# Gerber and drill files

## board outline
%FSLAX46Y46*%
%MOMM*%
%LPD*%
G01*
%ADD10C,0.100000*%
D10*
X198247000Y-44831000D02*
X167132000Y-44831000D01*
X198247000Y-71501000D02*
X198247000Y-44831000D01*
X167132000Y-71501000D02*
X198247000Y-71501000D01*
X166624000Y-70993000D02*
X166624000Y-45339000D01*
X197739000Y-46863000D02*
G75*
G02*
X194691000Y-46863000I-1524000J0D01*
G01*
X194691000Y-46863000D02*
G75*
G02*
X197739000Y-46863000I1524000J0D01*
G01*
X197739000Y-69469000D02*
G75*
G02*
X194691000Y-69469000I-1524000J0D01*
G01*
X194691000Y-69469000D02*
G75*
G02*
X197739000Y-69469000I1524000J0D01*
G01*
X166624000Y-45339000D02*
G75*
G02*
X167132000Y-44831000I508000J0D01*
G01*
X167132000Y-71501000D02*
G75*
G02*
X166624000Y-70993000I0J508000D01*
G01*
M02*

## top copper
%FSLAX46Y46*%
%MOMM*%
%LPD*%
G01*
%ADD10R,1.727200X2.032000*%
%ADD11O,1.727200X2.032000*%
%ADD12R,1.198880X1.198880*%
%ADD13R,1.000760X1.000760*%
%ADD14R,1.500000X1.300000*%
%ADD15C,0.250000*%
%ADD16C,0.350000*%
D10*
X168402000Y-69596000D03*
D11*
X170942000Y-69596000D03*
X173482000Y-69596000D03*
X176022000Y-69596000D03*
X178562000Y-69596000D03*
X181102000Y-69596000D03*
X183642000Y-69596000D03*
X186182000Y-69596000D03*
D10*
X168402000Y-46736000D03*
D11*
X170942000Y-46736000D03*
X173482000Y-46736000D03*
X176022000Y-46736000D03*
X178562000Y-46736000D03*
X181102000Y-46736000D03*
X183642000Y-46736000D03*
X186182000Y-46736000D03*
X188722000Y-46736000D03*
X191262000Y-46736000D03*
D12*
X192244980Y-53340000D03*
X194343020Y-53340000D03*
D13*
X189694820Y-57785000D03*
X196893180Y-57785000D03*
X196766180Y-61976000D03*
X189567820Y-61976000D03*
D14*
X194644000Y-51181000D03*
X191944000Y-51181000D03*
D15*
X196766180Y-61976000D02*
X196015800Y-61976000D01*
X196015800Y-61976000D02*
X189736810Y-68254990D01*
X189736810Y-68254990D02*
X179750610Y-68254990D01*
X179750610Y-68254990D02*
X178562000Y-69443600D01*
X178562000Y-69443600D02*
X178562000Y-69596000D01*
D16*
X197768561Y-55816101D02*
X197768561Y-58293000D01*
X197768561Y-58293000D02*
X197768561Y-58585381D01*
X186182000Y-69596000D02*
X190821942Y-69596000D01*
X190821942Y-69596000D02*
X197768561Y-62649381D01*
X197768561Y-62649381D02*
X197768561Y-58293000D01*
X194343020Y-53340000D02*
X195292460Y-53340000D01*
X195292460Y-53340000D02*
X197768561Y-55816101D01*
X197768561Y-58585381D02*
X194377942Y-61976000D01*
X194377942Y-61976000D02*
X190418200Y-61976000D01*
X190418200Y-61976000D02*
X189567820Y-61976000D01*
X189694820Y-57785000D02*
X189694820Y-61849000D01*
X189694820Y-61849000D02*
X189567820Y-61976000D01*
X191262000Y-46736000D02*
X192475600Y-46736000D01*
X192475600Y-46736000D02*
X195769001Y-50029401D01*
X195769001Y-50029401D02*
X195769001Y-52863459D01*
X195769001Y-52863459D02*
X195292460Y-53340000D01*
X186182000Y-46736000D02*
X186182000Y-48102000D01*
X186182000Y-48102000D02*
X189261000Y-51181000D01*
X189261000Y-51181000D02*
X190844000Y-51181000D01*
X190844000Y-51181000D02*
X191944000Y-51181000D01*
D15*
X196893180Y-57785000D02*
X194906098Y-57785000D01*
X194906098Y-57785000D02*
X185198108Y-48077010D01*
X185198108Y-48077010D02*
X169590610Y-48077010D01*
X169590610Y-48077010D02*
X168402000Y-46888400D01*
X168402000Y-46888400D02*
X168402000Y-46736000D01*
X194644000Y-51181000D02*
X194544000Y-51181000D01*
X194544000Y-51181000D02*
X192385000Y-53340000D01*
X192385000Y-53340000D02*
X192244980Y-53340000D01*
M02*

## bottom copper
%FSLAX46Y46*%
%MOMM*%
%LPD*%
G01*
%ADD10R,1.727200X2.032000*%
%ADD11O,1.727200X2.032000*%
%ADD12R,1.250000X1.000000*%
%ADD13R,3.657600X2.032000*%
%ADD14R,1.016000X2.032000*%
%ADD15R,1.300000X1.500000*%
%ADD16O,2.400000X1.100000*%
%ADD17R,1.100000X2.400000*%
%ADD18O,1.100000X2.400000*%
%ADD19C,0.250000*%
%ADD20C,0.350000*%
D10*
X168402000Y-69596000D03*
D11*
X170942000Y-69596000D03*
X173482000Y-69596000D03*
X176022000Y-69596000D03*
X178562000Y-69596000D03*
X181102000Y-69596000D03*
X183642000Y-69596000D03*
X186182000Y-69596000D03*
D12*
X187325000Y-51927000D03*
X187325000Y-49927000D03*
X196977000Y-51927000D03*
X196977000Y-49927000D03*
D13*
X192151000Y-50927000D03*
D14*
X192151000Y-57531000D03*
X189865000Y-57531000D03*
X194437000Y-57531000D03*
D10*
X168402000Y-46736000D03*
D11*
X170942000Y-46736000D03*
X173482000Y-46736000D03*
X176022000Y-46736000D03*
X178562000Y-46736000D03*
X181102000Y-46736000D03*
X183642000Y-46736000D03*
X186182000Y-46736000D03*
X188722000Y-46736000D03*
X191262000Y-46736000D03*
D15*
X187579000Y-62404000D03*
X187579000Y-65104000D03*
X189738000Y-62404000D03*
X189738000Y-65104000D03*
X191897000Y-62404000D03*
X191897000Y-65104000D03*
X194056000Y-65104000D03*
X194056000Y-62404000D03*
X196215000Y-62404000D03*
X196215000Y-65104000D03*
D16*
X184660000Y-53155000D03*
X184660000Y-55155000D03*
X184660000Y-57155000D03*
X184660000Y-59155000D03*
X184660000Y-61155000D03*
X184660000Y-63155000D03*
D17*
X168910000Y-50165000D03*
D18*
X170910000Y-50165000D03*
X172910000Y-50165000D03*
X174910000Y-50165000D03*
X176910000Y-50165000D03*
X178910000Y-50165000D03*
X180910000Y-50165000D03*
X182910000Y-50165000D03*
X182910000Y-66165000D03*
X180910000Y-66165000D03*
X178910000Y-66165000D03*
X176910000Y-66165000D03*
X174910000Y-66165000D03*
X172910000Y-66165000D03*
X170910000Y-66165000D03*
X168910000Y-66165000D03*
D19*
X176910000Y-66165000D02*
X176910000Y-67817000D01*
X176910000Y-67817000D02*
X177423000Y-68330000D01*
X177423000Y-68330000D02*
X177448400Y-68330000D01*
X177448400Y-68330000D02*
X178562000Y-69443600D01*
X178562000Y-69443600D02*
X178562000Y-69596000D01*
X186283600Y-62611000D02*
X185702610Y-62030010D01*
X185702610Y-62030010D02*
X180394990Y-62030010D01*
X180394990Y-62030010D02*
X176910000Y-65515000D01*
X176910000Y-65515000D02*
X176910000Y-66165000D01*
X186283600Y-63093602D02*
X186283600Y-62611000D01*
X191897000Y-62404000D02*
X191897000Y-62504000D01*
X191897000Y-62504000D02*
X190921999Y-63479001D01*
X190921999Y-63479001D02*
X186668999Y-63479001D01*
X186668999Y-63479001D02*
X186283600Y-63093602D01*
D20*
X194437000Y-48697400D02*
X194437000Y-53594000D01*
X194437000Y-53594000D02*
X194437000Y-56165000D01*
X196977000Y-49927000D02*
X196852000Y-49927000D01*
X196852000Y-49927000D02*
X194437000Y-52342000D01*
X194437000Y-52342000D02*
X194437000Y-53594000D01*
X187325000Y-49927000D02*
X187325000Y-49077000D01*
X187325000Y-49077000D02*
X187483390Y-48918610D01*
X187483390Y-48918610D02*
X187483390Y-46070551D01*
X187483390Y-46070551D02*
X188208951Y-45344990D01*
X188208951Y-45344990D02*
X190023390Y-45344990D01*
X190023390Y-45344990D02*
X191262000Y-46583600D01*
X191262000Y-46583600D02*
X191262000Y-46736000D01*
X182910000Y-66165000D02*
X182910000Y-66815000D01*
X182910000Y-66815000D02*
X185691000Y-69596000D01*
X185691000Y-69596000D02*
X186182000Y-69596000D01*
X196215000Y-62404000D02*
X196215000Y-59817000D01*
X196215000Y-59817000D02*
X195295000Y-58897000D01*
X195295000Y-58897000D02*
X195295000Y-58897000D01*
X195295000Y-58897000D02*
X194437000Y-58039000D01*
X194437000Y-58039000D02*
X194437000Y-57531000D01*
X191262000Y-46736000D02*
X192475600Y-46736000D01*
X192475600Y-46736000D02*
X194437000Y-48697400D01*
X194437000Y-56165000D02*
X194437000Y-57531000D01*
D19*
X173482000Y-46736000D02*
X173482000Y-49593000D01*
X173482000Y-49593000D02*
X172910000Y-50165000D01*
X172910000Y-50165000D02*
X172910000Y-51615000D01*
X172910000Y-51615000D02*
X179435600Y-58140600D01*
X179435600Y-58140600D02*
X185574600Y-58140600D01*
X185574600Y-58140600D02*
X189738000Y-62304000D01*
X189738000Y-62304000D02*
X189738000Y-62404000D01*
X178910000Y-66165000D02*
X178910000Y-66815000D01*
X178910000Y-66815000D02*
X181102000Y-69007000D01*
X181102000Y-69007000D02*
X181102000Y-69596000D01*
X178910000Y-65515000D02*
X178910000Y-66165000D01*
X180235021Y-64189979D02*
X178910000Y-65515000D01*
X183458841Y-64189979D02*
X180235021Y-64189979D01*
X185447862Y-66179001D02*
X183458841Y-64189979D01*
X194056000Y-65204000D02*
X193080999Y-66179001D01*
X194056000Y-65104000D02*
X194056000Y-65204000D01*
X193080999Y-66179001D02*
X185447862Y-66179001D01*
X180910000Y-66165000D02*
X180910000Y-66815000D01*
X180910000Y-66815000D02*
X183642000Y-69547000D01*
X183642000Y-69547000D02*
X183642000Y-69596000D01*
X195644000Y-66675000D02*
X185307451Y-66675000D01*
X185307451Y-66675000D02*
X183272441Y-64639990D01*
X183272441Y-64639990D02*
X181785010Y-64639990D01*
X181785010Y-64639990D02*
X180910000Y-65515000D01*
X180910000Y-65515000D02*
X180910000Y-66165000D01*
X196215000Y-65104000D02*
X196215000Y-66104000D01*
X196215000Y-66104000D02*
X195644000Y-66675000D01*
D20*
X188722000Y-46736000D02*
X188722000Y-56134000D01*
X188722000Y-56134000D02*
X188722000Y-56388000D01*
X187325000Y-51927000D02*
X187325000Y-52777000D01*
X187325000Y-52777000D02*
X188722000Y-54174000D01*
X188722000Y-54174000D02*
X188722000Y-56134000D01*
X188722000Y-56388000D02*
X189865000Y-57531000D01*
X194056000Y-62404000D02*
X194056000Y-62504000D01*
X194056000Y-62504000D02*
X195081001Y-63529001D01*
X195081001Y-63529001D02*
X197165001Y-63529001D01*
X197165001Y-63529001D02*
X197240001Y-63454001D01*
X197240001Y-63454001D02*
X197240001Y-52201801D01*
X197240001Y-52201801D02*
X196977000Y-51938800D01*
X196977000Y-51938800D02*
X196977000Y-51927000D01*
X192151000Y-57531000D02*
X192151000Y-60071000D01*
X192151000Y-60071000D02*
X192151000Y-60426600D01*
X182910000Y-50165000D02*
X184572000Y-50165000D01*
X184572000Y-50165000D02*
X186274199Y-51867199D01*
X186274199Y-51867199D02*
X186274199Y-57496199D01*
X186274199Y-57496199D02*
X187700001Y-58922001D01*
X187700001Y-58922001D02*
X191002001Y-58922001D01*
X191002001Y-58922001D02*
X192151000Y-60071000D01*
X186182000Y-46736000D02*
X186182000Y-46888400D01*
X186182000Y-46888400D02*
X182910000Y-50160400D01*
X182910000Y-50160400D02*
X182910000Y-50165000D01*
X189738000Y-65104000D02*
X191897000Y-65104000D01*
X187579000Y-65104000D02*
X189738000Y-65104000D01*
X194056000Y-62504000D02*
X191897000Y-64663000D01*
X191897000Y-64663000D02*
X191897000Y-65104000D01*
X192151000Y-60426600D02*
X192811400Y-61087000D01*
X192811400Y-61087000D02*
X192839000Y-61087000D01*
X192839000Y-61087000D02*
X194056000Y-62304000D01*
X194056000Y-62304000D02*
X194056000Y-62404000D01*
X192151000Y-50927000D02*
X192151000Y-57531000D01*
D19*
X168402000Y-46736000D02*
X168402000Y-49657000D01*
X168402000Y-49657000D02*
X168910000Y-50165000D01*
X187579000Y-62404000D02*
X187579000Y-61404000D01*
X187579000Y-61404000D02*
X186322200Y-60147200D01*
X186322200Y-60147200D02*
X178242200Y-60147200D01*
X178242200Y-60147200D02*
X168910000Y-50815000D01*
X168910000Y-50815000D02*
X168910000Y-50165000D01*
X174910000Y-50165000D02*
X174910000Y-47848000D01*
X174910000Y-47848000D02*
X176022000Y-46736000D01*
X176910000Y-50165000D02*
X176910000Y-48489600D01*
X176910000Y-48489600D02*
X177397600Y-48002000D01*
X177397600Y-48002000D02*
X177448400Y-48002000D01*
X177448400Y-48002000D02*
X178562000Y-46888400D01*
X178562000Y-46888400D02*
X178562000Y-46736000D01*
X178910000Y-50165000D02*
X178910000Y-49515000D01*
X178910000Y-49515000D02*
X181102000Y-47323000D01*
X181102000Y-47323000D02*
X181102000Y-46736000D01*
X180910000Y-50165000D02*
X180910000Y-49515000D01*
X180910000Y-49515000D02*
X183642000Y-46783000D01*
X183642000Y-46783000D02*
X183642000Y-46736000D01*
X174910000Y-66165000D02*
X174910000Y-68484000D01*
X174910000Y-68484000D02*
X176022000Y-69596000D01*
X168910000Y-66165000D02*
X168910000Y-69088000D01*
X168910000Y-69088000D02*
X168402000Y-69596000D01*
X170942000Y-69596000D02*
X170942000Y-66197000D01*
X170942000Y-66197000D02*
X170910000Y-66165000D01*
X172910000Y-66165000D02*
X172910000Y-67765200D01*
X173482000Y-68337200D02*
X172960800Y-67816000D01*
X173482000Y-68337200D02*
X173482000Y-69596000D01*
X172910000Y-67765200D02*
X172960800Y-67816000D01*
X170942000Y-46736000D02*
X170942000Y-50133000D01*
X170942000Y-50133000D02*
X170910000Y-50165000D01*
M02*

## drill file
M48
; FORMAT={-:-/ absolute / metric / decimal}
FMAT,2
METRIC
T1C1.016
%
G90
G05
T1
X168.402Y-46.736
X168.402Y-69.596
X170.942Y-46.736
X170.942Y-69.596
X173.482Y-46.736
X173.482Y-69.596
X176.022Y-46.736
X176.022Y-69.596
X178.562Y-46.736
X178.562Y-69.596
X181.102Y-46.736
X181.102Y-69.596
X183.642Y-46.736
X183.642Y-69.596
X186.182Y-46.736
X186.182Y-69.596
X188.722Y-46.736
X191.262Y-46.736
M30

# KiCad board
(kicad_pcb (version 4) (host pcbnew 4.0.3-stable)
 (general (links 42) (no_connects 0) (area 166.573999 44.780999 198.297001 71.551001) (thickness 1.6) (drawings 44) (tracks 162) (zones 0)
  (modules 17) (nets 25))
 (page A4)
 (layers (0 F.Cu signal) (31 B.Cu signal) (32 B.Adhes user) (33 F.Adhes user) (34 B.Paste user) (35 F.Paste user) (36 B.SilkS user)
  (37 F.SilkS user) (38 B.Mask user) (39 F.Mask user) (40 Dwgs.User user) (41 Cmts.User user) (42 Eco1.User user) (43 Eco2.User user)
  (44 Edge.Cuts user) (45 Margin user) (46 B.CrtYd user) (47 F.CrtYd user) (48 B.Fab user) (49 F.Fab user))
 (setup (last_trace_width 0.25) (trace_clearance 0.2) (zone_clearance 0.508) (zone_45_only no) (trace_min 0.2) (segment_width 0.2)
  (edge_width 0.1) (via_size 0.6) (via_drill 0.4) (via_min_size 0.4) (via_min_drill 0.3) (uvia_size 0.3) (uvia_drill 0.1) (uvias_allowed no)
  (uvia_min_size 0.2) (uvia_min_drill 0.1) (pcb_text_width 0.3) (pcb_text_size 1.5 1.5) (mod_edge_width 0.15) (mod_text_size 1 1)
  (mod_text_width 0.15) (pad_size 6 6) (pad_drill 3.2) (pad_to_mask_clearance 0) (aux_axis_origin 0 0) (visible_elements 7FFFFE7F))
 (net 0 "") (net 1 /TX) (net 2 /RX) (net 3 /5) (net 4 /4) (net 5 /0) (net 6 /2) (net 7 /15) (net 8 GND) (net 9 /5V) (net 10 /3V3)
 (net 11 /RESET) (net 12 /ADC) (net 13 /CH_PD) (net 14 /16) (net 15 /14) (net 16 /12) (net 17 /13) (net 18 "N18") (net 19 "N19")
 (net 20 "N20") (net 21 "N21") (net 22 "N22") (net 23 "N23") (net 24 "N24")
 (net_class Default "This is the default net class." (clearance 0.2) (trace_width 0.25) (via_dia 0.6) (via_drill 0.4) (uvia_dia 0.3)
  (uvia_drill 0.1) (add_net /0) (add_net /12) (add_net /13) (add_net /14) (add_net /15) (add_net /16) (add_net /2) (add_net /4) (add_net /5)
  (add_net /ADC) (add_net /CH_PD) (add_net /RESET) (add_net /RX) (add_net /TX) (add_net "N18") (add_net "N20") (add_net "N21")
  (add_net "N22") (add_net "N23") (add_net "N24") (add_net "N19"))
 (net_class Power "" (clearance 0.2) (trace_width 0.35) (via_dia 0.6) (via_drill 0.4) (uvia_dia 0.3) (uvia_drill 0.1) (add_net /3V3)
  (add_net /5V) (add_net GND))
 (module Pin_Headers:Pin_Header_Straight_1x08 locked (layer B.Cu) (at 168.402 69.596 270)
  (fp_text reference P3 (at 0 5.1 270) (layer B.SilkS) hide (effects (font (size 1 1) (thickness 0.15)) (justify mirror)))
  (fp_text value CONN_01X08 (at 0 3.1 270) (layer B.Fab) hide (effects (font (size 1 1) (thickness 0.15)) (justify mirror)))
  (pad 1 thru_hole rect (at 0 0 270) (size 2.032 1.7272) (drill 1.016) (layers *.Cu *.Mask B.SilkS) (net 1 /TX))
  (pad 2 thru_hole oval (at 0 -2.54 270) (size 2.032 1.7272) (drill 1.016) (layers *.Cu *.Mask B.SilkS) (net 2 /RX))
  (pad 3 thru_hole oval (at 0 -5.08 270) (size 2.032 1.7272) (drill 1.016) (layers *.Cu *.Mask B.SilkS) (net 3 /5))
  (pad 4 thru_hole oval (at 0 -7.62 270) (size 2.032 1.7272) (drill 1.016) (layers *.Cu *.Mask B.SilkS) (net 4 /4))
  (pad 5 thru_hole oval (at 0 -10.16 270) (size 2.032 1.7272) (drill 1.016) (layers *.Cu *.Mask B.SilkS) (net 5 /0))
  (pad 6 thru_hole oval (at 0 -12.7 270) (size 2.032 1.7272) (drill 1.016) (layers *.Cu *.Mask B.SilkS) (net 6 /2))
  (pad 7 thru_hole oval (at 0 -15.24 270) (size 2.032 1.7272) (drill 1.016) (layers *.Cu *.Mask B.SilkS) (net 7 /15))
  (pad 8 thru_hole oval (at 0 -17.78 270) (size 2.032 1.7272) (drill 1.016) (layers *.Cu *.Mask B.SilkS) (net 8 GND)))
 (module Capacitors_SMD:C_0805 (layer B.Cu) (at 187.325 50.927 90)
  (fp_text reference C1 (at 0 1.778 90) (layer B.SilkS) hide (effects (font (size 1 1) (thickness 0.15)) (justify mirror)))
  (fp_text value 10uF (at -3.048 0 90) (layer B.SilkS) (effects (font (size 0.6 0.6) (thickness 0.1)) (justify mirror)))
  (pad 1 smd rect (at -1 0 90) (size 1 1.25) (layers B.Cu B.Paste B.Mask) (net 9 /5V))
  (pad 2 smd rect (at 1 0 90) (size 1 1.25) (layers B.Cu B.Paste B.Mask) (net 8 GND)))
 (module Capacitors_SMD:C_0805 (layer B.Cu) (at 196.977 50.927 90)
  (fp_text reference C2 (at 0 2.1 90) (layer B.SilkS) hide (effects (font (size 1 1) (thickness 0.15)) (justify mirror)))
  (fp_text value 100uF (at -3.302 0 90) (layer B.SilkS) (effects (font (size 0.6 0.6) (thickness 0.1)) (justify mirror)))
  (pad 1 smd rect (at -1 0 90) (size 1 1.25) (layers B.Cu B.Paste B.Mask) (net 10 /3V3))
  (pad 2 smd rect (at 1 0 90) (size 1 1.25) (layers B.Cu B.Paste B.Mask) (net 8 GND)))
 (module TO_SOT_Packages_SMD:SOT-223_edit (layer B.Cu) (at 192.151 54.229 180)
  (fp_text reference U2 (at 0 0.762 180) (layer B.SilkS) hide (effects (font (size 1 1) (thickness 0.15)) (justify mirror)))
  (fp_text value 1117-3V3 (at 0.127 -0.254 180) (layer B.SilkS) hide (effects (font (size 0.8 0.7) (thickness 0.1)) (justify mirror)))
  (pad 2 smd rect (at 0 3.302 180) (size 3.6576 2.032) (layers B.Cu B.Paste B.Mask) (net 10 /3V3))
  (pad 2 smd rect (at 0 -3.302 180) (size 1.016 2.032) (layers B.Cu B.Paste B.Mask) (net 10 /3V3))
  (pad 3 smd rect (at 2.286 -3.302 180) (size 1.016 2.032) (layers B.Cu B.Paste B.Mask) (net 9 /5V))
  (pad 1 smd rect (at -2.286 -3.302 180) (size 1.016 2.032) (layers B.Cu B.Paste B.Mask) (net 8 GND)))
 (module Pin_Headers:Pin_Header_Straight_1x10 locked (layer B.Cu) (at 168.402 46.736 270)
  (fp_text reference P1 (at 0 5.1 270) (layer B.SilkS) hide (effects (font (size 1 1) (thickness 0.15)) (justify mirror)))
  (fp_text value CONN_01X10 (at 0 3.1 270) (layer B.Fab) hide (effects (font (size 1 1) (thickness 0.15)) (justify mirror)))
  (pad 1 thru_hole rect (at 0 0 270) (size 2.032 1.7272) (drill 1.016) (layers *.Cu *.Mask B.SilkS) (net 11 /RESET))
  (pad 2 thru_hole oval (at 0 -2.54 270) (size 2.032 1.7272) (drill 1.016) (layers *.Cu *.Mask B.SilkS) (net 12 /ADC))
  (pad 3 thru_hole oval (at 0 -5.08 270) (size 2.032 1.7272) (drill 1.016) (layers *.Cu *.Mask B.SilkS) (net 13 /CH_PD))
  (pad 4 thru_hole oval (at 0 -7.62 270) (size 2.032 1.7272) (drill 1.016) (layers *.Cu *.Mask B.SilkS) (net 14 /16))
  (pad 5 thru_hole oval (at 0 -10.16 270) (size 2.032 1.7272) (drill 1.016) (layers *.Cu *.Mask B.SilkS) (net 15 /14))
  (pad 6 thru_hole oval (at 0 -12.7 270) (size 2.032 1.7272) (drill 1.016) (layers *.Cu *.Mask B.SilkS) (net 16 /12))
  (pad 7 thru_hole oval (at 0 -15.24 270) (size 2.032 1.7272) (drill 1.016) (layers *.Cu *.Mask B.SilkS) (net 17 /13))
  (pad 8 thru_hole oval (at 0 -17.78 270) (size 2.032 1.7272) (drill 1.016) (layers *.Cu *.Mask B.SilkS) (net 10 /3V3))
  (pad 9 thru_hole oval (at 0 -20.32 270) (size 2.032 1.7272) (drill 1.016) (layers *.Cu *.Mask B.SilkS) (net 9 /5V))
  (pad 10 thru_hole oval (at 0 -22.86 270) (size 2.032 1.7272) (drill 1.016) (layers *.Cu *.Mask B.SilkS) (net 8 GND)))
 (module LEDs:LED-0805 (layer F.Cu) (at 193.294 53.34 180)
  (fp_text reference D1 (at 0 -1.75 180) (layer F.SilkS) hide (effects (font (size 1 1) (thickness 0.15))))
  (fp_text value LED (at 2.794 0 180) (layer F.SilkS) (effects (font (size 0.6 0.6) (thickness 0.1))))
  (pad 2 smd rect (at 1.04902 0) (size 1.19888 1.19888) (layers F.Cu F.Paste F.Mask) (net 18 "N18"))
  (pad 1 smd rect (at -1.04902 0) (size 1.19888 1.19888) (layers F.Cu F.Paste F.Mask) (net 8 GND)))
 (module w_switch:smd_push (layer F.Cu) (at 193.294 57.785) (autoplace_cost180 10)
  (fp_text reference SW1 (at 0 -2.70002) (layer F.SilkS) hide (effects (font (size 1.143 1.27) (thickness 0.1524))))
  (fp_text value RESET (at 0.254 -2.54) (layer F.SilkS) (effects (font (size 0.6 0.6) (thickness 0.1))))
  (pad 1 smd rect (at -3.59918 0) (size 1.00076 1.00076) (layers F.Cu F.Paste F.Mask) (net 8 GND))
  (pad 2 smd rect (at 3.59918 0) (size 1.00076 1.00076) (layers F.Cu F.Paste F.Mask) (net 11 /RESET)))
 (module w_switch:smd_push (layer F.Cu) (at 193.167 61.976 180) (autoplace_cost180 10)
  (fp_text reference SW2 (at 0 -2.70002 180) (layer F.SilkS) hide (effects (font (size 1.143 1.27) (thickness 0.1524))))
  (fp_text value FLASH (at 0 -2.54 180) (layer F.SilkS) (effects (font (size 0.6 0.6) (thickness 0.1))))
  (pad 1 smd rect (at -3.59918 0 180) (size 1.00076 1.00076) (layers F.Cu F.Paste F.Mask) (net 5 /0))
  (pad 2 smd rect (at 3.59918 0 180) (size 1.00076 1.00076) (layers F.Cu F.Paste F.Mask) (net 8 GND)))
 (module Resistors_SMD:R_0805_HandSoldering (layer B.Cu) (at 187.579 63.754 270)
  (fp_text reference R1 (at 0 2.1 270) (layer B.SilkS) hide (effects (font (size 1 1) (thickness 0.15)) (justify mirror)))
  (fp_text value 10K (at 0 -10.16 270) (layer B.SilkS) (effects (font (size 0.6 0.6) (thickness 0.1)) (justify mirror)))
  (pad 1 smd rect (at -1.35 0 270) (size 1.5 1.3) (layers B.Cu B.Paste B.Mask) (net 11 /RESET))
  (pad 2 smd rect (at 1.35 0 270) (size 1.5 1.3) (layers B.Cu B.Paste B.Mask) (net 10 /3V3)))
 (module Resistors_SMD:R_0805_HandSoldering (layer B.Cu) (at 189.738 63.754 270)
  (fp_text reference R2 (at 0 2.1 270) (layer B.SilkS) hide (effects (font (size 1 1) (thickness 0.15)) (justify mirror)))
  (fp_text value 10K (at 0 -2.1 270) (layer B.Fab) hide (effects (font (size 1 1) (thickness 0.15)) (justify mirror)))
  (pad 1 smd rect (at -1.35 0 270) (size 1.5 1.3) (layers B.Cu B.Paste B.Mask) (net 13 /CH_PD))
  (pad 2 smd rect (at 1.35 0 270) (size 1.5 1.3) (layers B.Cu B.Paste B.Mask) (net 10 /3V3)))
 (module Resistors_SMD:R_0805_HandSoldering (layer B.Cu) (at 191.897 63.754 270)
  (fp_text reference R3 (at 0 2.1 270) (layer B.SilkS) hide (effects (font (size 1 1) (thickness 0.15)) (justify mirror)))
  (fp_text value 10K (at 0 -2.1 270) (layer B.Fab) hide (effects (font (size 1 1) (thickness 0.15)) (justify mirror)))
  (pad 1 smd rect (at -1.35 0 270) (size 1.5 1.3) (layers B.Cu B.Paste B.Mask) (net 5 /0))
  (pad 2 smd rect (at 1.35 0 270) (size 1.5 1.3) (layers B.Cu B.Paste B.Mask) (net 10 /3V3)))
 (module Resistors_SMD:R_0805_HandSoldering (layer B.Cu) (at 194.056 63.754 90)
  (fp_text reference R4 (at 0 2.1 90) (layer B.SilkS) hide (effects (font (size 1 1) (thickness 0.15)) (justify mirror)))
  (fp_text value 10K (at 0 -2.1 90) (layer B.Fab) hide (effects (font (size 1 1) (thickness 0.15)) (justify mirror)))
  (pad 1 smd rect (at -1.35 0 90) (size 1.5 1.3) (layers B.Cu B.Paste B.Mask) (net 6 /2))
  (pad 2 smd rect (at 1.35 0 90) (size 1.5 1.3) (layers B.Cu B.Paste B.Mask) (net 10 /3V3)))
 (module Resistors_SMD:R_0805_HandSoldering (layer B.Cu) (at 196.215 63.754 270)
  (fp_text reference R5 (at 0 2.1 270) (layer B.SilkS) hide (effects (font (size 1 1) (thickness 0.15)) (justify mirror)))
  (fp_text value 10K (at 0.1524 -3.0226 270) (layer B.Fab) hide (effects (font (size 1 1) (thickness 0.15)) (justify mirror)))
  (pad 1 smd rect (at -1.35 0 270) (size 1.5 1.3) (layers B.Cu B.Paste B.Mask) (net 8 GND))
  (pad 2 smd rect (at 1.35 0 270) (size 1.5 1.3) (layers B.Cu B.Paste B.Mask) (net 7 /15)))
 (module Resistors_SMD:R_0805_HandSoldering (layer F.Cu) (at 193.294 51.181 180)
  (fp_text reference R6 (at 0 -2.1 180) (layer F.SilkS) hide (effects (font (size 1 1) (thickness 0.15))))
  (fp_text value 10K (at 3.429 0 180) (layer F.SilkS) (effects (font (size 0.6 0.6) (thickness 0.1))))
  (pad 1 smd rect (at -1.35 0 180) (size 1.5 1.3) (layers F.Cu F.Paste F.Mask) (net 18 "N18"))
  (pad 2 smd rect (at 1.35 0 180) (size 1.5 1.3) (layers F.Cu F.Paste F.Mask) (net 10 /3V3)))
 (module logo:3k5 (layer F.Cu) (at 177.546 56.515)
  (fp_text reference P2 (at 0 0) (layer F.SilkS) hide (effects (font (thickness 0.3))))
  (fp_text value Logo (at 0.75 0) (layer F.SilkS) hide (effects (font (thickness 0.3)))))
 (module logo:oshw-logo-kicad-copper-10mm (layer F.Cu) (at 190.627 67.564)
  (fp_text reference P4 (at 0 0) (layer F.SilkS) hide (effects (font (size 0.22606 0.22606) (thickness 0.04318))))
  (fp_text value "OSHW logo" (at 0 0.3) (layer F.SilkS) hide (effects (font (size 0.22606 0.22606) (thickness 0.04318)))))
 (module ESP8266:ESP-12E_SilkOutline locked (layer B.Cu) (at 168.91 50.165 270)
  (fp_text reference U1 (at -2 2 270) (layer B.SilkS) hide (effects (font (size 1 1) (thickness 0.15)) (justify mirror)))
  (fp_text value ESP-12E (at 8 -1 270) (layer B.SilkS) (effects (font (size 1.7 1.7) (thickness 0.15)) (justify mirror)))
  (pad 9 smd oval (at 2.99 -15.75 180) (size 2.4 1.1) (layers B.Cu B.Paste B.Mask) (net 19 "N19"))
  (pad 10 smd oval (at 4.99 -15.75 180) (size 2.4 1.1) (layers B.Cu B.Paste B.Mask) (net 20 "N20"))
  (pad 11 smd oval (at 6.99 -15.75 180) (size 2.4 1.1) (layers B.Cu B.Paste B.Mask) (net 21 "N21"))
  (pad 12 smd oval (at 8.99 -15.75 180) (size 2.4 1.1) (layers B.Cu B.Paste B.Mask) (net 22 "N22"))
  (pad 13 smd oval (at 10.99 -15.75 180) (size 2.4 1.1) (layers B.Cu B.Paste B.Mask) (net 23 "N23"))
  (pad 14 smd oval (at 12.99 -15.75 180) (size 2.4 1.1) (layers B.Cu B.Paste B.Mask) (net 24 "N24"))
  (pad 1 smd rect (at 0 0 270) (size 2.4 1.1) (layers B.Cu B.Paste B.Mask) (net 11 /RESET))
  (pad 2 smd oval (at 0 -2 270) (size 2.4 1.1) (layers B.Cu B.Paste B.Mask) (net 12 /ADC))
  (pad 3 smd oval (at 0 -4 270) (size 2.4 1.1) (layers B.Cu B.Paste B.Mask) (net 13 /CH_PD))
  (pad 4 smd oval (at 0 -6 270) (size 2.4 1.1) (layers B.Cu B.Paste B.Mask) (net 14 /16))
  (pad 5 smd oval (at 0 -8 270) (size 2.4 1.1) (layers B.Cu B.Paste B.Mask) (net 15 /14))
  (pad 6 smd oval (at 0 -10 270) (size 2.4 1.1) (layers B.Cu B.Paste B.Mask) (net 16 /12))
  (pad 7 smd oval (at 0 -12 270) (size 2.4 1.1) (layers B.Cu B.Paste B.Mask) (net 17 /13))
  (pad 8 smd oval (at 0 -14 270) (size 2.4 1.1) (layers B.Cu B.Paste B.Mask) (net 10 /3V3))
  (pad 15 smd oval (at 16 -14 270) (size 2.4 1.1) (layers B.Cu B.Paste B.Mask) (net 8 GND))
  (pad 16 smd oval (at 16 -12 270) (size 2.4 1.1) (layers B.Cu B.Paste B.Mask) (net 7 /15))
  (pad 17 smd oval (at 16 -10 270) (size 2.4 1.1) (layers B.Cu B.Paste B.Mask) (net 6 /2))
  (pad 18 smd oval (at 16 -8 270) (size 2.4 1.1) (layers B.Cu B.Paste B.Mask) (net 5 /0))
  (pad 19 smd oval (at 16 -6 270) (size 2.4 1.1) (layers B.Cu B.Paste B.Mask) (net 4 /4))
  (pad 20 smd oval (at 16 -4 270) (size 2.4 1.1) (layers B.Cu B.Paste B.Mask) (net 3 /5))
  (pad 21 smd oval (at 16 -2 270) (size 2.4 1.1) (layers B.Cu B.Paste B.Mask) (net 2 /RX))
  (pad 22 smd oval (at 16 0 270) (size 2.4 1.1) (layers B.Cu B.Paste B.Mask) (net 1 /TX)))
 (gr_line (start 198.247 44.831) (end 167.132 44.831) (angle 90) (layer Edge.Cuts) (width 0.1))
 (gr_line (start 198.247 71.501) (end 198.247 44.831) (angle 90) (layer Edge.Cuts) (width 0.1))
 (gr_line (start 167.132 71.501) (end 198.247 71.501) (angle 90) (layer Edge.Cuts) (width 0.1))
 (gr_line (start 166.624 70.993) (end 166.624 45.339) (angle 90) (layer Edge.Cuts) (width 0.1))
 (gr_circle (center 196.215 46.863) (end 196.215 45.339) (layer Edge.Cuts) (width 0.1))
 (gr_circle (center 196.215 69.469) (end 196.215 67.945) (layer Edge.Cuts) (width 0.1))
 (gr_arc (start 167.132 45.339) (end 166.624 45.339) (angle 90) (layer Edge.Cuts) (width 0.1))
 (gr_arc (start 167.132 70.993) (end 167.132 71.501) (angle 90) (layer Edge.Cuts) (width 0.1))
 (segment (start 196.76618 61.976) (end 196.0158 61.976) (width 0.25) (layer F.Cu) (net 5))
 (segment (start 196.0158 61.976) (end 189.73681 68.25499) (width 0.25) (layer F.Cu) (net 5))
 (segment (start 189.73681 68.25499) (end 179.75061 68.25499) (width 0.25) (layer F.Cu) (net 5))
 (segment (start 179.75061 68.25499) (end 178.562 69.4436) (width 0.25) (layer F.Cu) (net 5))
 (segment (start 178.562 69.4436) (end 178.562 69.596) (width 0.25) (layer F.Cu) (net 5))
 (segment (start 176.91 66.165) (end 176.91 67.817) (width 0.25) (layer B.Cu) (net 5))
 (segment (start 176.91 67.817) (end 177.423 68.33) (width 0.25) (layer B.Cu) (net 5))
 (segment (start 177.423 68.33) (end 177.4484 68.33) (width 0.25) (layer B.Cu) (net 5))
 (segment (start 177.4484 68.33) (end 178.562 69.4436) (width 0.25) (layer B.Cu) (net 5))
 (segment (start 178.562 69.4436) (end 178.562 69.596) (width 0.25) (layer B.Cu) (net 5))
 (segment (start 186.2836 62.611) (end 185.70261 62.03001) (width 0.25) (layer B.Cu) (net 5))
 (segment (start 185.70261 62.03001) (end 180.39499 62.03001) (width 0.25) (layer B.Cu) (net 5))
 (segment (start 180.39499 62.03001) (end 176.91 65.515) (width 0.25) (layer B.Cu) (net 5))
 (segment (start 176.91 65.515) (end 176.91 66.165) (width 0.25) (layer B.Cu) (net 5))
 (segment (start 186.2836 63.093602) (end 186.2836 62.611) (width 0.25) (layer B.Cu) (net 5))
 (segment (start 191.897 62.404) (end 191.897 62.504) (width 0.25) (layer B.Cu) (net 5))
 (segment (start 191.897 62.504) (end 190.921999 63.479001) (width 0.25) (layer B.Cu) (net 5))
 (segment (start 190.921999 63.479001) (end 186.668999 63.479001) (width 0.25) (layer B.Cu) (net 5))
 (segment (start 186.668999 63.479001) (end 186.2836 63.093602) (width 0.25) (layer B.Cu) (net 5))
 (segment (start 194.437 48.6974) (end 194.437 53.594) (width 0.35) (layer B.Cu) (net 8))
 (segment (start 194.437 53.594) (end 194.437 56.165) (width 0.35) (layer B.Cu) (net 8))
 (segment (start 196.977 49.927) (end 196.852 49.927) (width 0.35) (layer B.Cu) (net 8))
 (segment (start 196.852 49.927) (end 194.437 52.342) (width 0.35) (layer B.Cu) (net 8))
 (segment (start 194.437 52.342) (end 194.437 53.594) (width 0.35) (layer B.Cu) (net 8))
 (segment (start 197.768561 55.816101) (end 197.768561 58.293) (width 0.35) (layer F.Cu) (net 8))
 (segment (start 197.768561 58.293) (end 197.768561 58.585381) (width 0.35) (layer F.Cu) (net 8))
 (segment (start 186.182 69.596) (end 190.821942 69.596) (width 0.35) (layer F.Cu) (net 8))
 (segment (start 190.821942 69.596) (end 197.768561 62.649381) (width 0.35) (layer F.Cu) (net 8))
 (segment (start 197.768561 62.649381) (end 197.768561 58.293) (width 0.35) (layer F.Cu) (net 8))
 (segment (start 187.325 49.927) (end 187.325 49.077) (width 0.35) (layer B.Cu) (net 8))
 (segment (start 187.325 49.077) (end 187.48339 48.91861) (width 0.35) (layer B.Cu) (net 8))
 (segment (start 187.48339 48.91861) (end 187.48339 46.070551) (width 0.35) (layer B.Cu) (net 8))
 (segment (start 187.48339 46.070551) (end 188.208951 45.34499) (width 0.35) (layer B.Cu) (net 8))
 (segment (start 188.208951 45.34499) (end 190.02339 45.34499) (width 0.35) (layer B.Cu) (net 8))
 (segment (start 190.02339 45.34499) (end 191.262 46.5836) (width 0.35) (layer B.Cu) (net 8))
 (segment (start 191.262 46.5836) (end 191.262 46.736) (width 0.35) (layer B.Cu) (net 8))
 (segment (start 194.34302 53.34) (end 195.29246 53.34) (width 0.35) (layer F.Cu) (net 8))
 (segment (start 195.29246 53.34) (end 197.768561 55.816101) (width 0.35) (layer F.Cu) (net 8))
 (segment (start 197.768561 58.585381) (end 194.377942 61.976) (width 0.35) (layer F.Cu) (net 8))
 (segment (start 194.377942 61.976) (end 190.4182 61.976) (width 0.35) (layer F.Cu) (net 8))
 (segment (start 190.4182 61.976) (end 189.56782 61.976) (width 0.35) (layer F.Cu) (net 8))
 (segment (start 189.69482 57.785) (end 189.69482 61.849) (width 0.35) (layer F.Cu) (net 8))
 (segment (start 189.69482 61.849) (end 189.56782 61.976) (width 0.35) (layer F.Cu) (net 8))
 (segment (start 191.262 46.736) (end 192.4756 46.736) (width 0.35) (layer F.Cu) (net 8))
 (segment (start 192.4756 46.736) (end 195.769001 50.029401) (width 0.35) (layer F.Cu) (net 8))
 (segment (start 195.769001 50.029401) (end 195.769001 52.863459) (width 0.35) (layer F.Cu) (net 8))
 (segment (start 195.769001 52.863459) (end 195.29246 53.34) (width 0.35) (layer F.Cu) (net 8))
 (segment (start 182.91 66.165) (end 182.91 66.815) (width 0.35) (layer B.Cu) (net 8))
 (segment (start 182.91 66.815) (end 185.691 69.596) (width 0.35) (layer B.Cu) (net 8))
 (segment (start 185.691 69.596) (end 186.182 69.596) (width 0.35) (layer B.Cu) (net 8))
 (segment (start 196.215 62.404) (end 196.215 59.817) (width 0.35) (layer B.Cu) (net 8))
 (segment (start 196.215 59.817) (end 195.295 58.897) (width 0.35) (layer B.Cu) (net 8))
 (segment (start 195.295 58.897) (end 195.295 58.897) (width 0.35) (layer B.Cu) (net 8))
 (segment (start 195.295 58.897) (end 194.437 58.039) (width 0.35) (layer B.Cu) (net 8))
 (segment (start 194.437 58.039) (end 194.437 57.531) (width 0.35) (layer B.Cu) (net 8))
 (segment (start 191.262 46.736) (end 192.4756 46.736) (width 0.35) (layer B.Cu) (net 8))
 (segment (start 192.4756 46.736) (end 194.437 48.6974) (width 0.35) (layer B.Cu) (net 8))
 (segment (start 194.437 56.165) (end 194.437 57.531) (width 0.35) (layer B.Cu) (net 8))
 (segment (start 173.482 46.736) (end 173.482 49.593) (width 0.25) (layer B.Cu) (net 13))
 (segment (start 173.482 49.593) (end 172.91 50.165) (width 0.25) (layer B.Cu) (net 13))
 (segment (start 172.91 50.165) (end 172.91 51.615) (width 0.25) (layer B.Cu) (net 13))
 (segment (start 172.91 51.615) (end 179.4356 58.1406) (width 0.25) (layer B.Cu) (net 13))
 (segment (start 179.4356 58.1406) (end 185.5746 58.1406) (width 0.25) (layer B.Cu) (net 13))
 (segment (start 185.5746 58.1406) (end 189.738 62.304) (width 0.25) (layer B.Cu) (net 13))
 (segment (start 189.738 62.304) (end 189.738 62.404) (width 0.25) (layer B.Cu) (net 13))
 (segment (start 178.91 66.165) (end 178.91 66.815) (width 0.25) (layer B.Cu) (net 6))
 (segment (start 178.91 66.815) (end 181.102 69.007) (width 0.25) (layer B.Cu) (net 6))
 (segment (start 181.102 69.007) (end 181.102 69.596) (width 0.25) (layer B.Cu) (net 6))
 (segment (start 178.91 65.515) (end 178.91 66.165) (width 0.25) (layer B.Cu) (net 6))
 (segment (start 180.235021 64.189979) (end 178.91 65.515) (width 0.25) (layer B.Cu) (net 6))
 (segment (start 183.458841 64.189979) (end 180.235021 64.189979) (width 0.25) (layer B.Cu) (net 6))
 (segment (start 185.447862 66.179001) (end 183.458841 64.189979) (width 0.25) (layer B.Cu) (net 6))
 (segment (start 194.056 65.204) (end 193.080999 66.179001) (width 0.25) (layer B.Cu) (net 6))
 (segment (start 194.056 65.104) (end 194.056 65.204) (width 0.25) (layer B.Cu) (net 6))
 (segment (start 193.080999 66.179001) (end 185.447862 66.179001) (width 0.25) (layer B.Cu) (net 6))
 (segment (start 180.91 66.165) (end 180.91 66.815) (width 0.25) (layer B.Cu) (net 7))
 (segment (start 180.91 66.815) (end 183.642 69.547) (width 0.25) (layer B.Cu) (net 7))
 (segment (start 183.642 69.547) (end 183.642 69.596) (width 0.25) (layer B.Cu) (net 7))
 (segment (start 195.644 66.675) (end 185.307451 66.675) (width 0.25) (layer B.Cu) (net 7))
 (segment (start 185.307451 66.675) (end 183.272441 64.63999) (width 0.25) (layer B.Cu) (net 7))
 (segment (start 183.272441 64.63999) (end 181.78501 64.63999) (width 0.25) (layer B.Cu) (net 7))
 (segment (start 181.78501 64.63999) (end 180.91 65.515) (width 0.25) (layer B.Cu) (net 7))
 (segment (start 180.91 65.515) (end 180.91 66.165) (width 0.25) (layer B.Cu) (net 7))
 (segment (start 196.215 65.104) (end 196.215 66.104) (width 0.25) (layer B.Cu) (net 7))
 (segment (start 196.215 66.104) (end 195.644 66.675) (width 0.25) (layer B.Cu) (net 7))
 (segment (start 188.722 46.736) (end 188.722 56.134) (width 0.35) (layer B.Cu) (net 9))
 (segment (start 188.722 56.134) (end 188.722 56.388) (width 0.35) (layer B.Cu) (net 9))
 (segment (start 187.325 51.927) (end 187.325 52.777) (width 0.35) (layer B.Cu) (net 9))
 (segment (start 187.325 52.777) (end 188.722 54.174) (width 0.35) (layer B.Cu) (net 9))
 (segment (start 188.722 54.174) (end 188.722 56.134) (width 0.35) (layer B.Cu) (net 9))
 (segment (start 188.722 56.388) (end 189.865 57.531) (width 0.35) (layer B.Cu) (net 9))
 (segment (start 194.056 62.404) (end 194.056 62.504) (width 0.35) (layer B.Cu) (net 10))
 (segment (start 194.056 62.504) (end 195.081001 63.529001) (width 0.35) (layer B.Cu) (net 10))
 (segment (start 195.081001 63.529001) (end 197.165001 63.529001) (width 0.35) (layer B.Cu) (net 10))
 (segment (start 197.165001 63.529001) (end 197.240001 63.454001) (width 0.35) (layer B.Cu) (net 10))
 (segment (start 197.240001 63.454001) (end 197.240001 52.201801) (width 0.35) (layer B.Cu) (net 10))
 (segment (start 197.240001 52.201801) (end 196.977 51.9388) (width 0.35) (layer B.Cu) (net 10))
 (segment (start 196.977 51.9388) (end 196.977 51.927) (width 0.35) (layer B.Cu) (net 10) (status 800000))
 (segment (start 192.151 57.531) (end 192.151 60.071) (width 0.35) (layer B.Cu) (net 10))
 (segment (start 192.151 60.071) (end 192.151 60.4266) (width 0.35) (layer B.Cu) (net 10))
 (segment (start 182.91 50.165) (end 184.572 50.165) (width 0.35) (layer B.Cu) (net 10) (status 400000))
 (segment (start 184.572 50.165) (end 186.274199 51.867199) (width 0.35) (layer B.Cu) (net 10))
 (segment (start 186.274199 51.867199) (end 186.274199 57.496199) (width 0.35) (layer B.Cu) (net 10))
 (segment (start 186.274199 57.496199) (end 187.700001 58.922001) (width 0.35) (layer B.Cu) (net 10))
 (segment (start 187.700001 58.922001) (end 191.002001 58.922001) (width 0.35) (layer B.Cu) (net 10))
 (segment (start 191.002001 58.922001) (end 192.151 60.071) (width 0.35) (layer B.Cu) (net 10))
 (segment (start 186.182 46.736) (end 186.182 48.102) (width 0.35) (layer F.Cu) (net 10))
 (segment (start 186.182 48.102) (end 189.261 51.181) (width 0.35) (layer F.Cu) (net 10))
 (segment (start 189.261 51.181) (end 190.844 51.181) (width 0.35) (layer F.Cu) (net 10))
 (segment (start 190.844 51.181) (end 191.944 51.181) (width 0.35) (layer F.Cu) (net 10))
 (segment (start 186.182 46.736) (end 186.182 46.8884) (width 0.35) (layer B.Cu) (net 10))
 (segment (start 186.182 46.8884) (end 182.91 50.1604) (width 0.35) (layer B.Cu) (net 10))
 (segment (start 182.91 50.1604) (end 182.91 50.165) (width 0.35) (layer B.Cu) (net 10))
 (segment (start 189.738 65.104) (end 191.897 65.104) (width 0.35) (layer B.Cu) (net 10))
 (segment (start 187.579 65.104) (end 189.738 65.104) (width 0.35) (layer B.Cu) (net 10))
 (segment (start 194.056 62.504) (end 191.897 64.663) (width 0.35) (layer B.Cu) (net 10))
 (segment (start 191.897 64.663) (end 191.897 65.104) (width 0.35) (layer B.Cu) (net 10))
 (segment (start 192.151 60.4266) (end 192.8114 61.087) (width 0.35) (layer B.Cu) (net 10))
 (segment (start 192.8114 61.087) (end 192.839 61.087) (width 0.35) (layer B.Cu) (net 10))
 (segment (start 192.839 61.087) (end 194.056 62.304) (width 0.35) (layer B.Cu) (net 10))
 (segment (start 194.056 62.304) (end 194.056 62.404) (width 0.35) (layer B.Cu) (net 10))
 (segment (start 192.151 50.927) (end 192.151 57.531) (width 0.35) (layer B.Cu) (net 10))
 (segment (start 196.89318 57.785) (end 194.906098 57.785) (width 0.25) (layer F.Cu) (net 11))
 (segment (start 194.906098 57.785) (end 185.198108 48.07701) (width 0.25) (layer F.Cu) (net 11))
 (segment (start 185.198108 48.07701) (end 169.59061 48.07701) (width 0.25) (layer F.Cu) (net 11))
 (segment (start 169.59061 48.07701) (end 168.402 46.8884) (width 0.25) (layer F.Cu) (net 11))
 (segment (start 168.402 46.8884) (end 168.402 46.736) (width 0.25) (layer F.Cu) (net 11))
 (segment (start 168.402 46.736) (end 168.402 49.657) (width 0.25) (layer B.Cu) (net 11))
 (segment (start 168.402 49.657) (end 168.91 50.165) (width 0.25) (layer B.Cu) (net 11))
 (segment (start 187.579 62.404) (end 187.579 61.404) (width 0.25) (layer B.Cu) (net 11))
 (segment (start 187.579 61.404) (end 186.3222 60.1472) (width 0.25) (layer B.Cu) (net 11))
 (segment (start 186.3222 60.1472) (end 178.2422 60.1472) (width 0.25) (layer B.Cu) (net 11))
 (segment (start 178.2422 60.1472) (end 168.91 50.815) (width 0.25) (layer B.Cu) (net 11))
 (segment (start 168.91 50.815) (end 168.91 50.165) (width 0.25) (layer B.Cu) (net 11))
 (segment (start 174.91 50.165) (end 174.91 47.848) (width 0.25) (layer B.Cu) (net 14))
 (segment (start 174.91 47.848) (end 176.022 46.736) (width 0.25) (layer B.Cu) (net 14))
 (segment (start 176.91 50.165) (end 176.91 48.4896) (width 0.25) (layer B.Cu) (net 15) (status 400000))
 (segment (start 176.91 48.4896) (end 177.3976 48.002) (width 0.25) (layer B.Cu) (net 15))
 (segment (start 177.3976 48.002) (end 177.4484 48.002) (width 0.25) (layer B.Cu) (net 15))
 (segment (start 177.4484 48.002) (end 178.562 46.8884) (width 0.25) (layer B.Cu) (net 15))
 (segment (start 178.562 46.8884) (end 178.562 46.736) (width 0.25) (layer B.Cu) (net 15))
 (segment (start 178.91 50.165) (end 178.91 49.515) (width 0.25) (layer B.Cu) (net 16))
 (segment (start 178.91 49.515) (end 181.102 47.323) (width 0.25) (layer B.Cu) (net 16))
 (segment (start 181.102 47.323) (end 181.102 46.736) (width 0.25) (layer B.Cu) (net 16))
 (segment (start 180.91 50.165) (end 180.91 49.515) (width 0.25) (layer B.Cu) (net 17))
 (segment (start 180.91 49.515) (end 183.642 46.783) (width 0.25) (layer B.Cu) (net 17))
 (segment (start 183.642 46.783) (end 183.642 46.736) (width 0.25) (layer B.Cu) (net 17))
 (segment (start 174.91 66.165) (end 174.91 68.484) (width 0.25) (layer B.Cu) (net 4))
 (segment (start 174.91 68.484) (end 176.022 69.596) (width 0.25) (layer B.Cu) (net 4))
 (segment (start 168.91 66.165) (end 168.91 69.088) (width 0.25) (layer B.Cu) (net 1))
 (segment (start 168.91 69.088) (end 168.402 69.596) (width 0.25) (layer B.Cu) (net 1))
 (segment (start 170.942 69.596) (end 170.942 66.197) (width 0.25) (layer B.Cu) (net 2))
 (segment (start 170.942 66.197) (end 170.91 66.165) (width 0.25) (layer B.Cu) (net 2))
 (segment (start 172.91 66.165) (end 172.91 67.7652) (width 0.25) (layer B.Cu) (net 3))
 (segment (start 173.482 68.3372) (end 172.9608 67.816) (width 0.25) (layer B.Cu) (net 3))
 (segment (start 173.482 68.3372) (end 173.482 69.596) (width 0.25) (layer B.Cu) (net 3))
 (segment (start 172.91 67.7652) (end 172.9608 67.816) (width 0.25) (layer B.Cu) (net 3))
 (segment (start 170.942 46.736) (end 170.942 50.133) (width 0.25) (layer B.Cu) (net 12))
 (segment (start 170.942 50.133) (end 170.91 50.165) (width 0.25) (layer B.Cu) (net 12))
 (segment (start 194.644 51.181) (end 194.544 51.181) (width 0.25) (layer F.Cu) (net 18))
 (segment (start 194.544 51.181) (end 192.385 53.34) (width 0.25) (layer F.Cu) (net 18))
 (segment (start 192.385 53.34) (end 192.24498 53.34) (width 0.25) (layer F.Cu) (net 18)))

